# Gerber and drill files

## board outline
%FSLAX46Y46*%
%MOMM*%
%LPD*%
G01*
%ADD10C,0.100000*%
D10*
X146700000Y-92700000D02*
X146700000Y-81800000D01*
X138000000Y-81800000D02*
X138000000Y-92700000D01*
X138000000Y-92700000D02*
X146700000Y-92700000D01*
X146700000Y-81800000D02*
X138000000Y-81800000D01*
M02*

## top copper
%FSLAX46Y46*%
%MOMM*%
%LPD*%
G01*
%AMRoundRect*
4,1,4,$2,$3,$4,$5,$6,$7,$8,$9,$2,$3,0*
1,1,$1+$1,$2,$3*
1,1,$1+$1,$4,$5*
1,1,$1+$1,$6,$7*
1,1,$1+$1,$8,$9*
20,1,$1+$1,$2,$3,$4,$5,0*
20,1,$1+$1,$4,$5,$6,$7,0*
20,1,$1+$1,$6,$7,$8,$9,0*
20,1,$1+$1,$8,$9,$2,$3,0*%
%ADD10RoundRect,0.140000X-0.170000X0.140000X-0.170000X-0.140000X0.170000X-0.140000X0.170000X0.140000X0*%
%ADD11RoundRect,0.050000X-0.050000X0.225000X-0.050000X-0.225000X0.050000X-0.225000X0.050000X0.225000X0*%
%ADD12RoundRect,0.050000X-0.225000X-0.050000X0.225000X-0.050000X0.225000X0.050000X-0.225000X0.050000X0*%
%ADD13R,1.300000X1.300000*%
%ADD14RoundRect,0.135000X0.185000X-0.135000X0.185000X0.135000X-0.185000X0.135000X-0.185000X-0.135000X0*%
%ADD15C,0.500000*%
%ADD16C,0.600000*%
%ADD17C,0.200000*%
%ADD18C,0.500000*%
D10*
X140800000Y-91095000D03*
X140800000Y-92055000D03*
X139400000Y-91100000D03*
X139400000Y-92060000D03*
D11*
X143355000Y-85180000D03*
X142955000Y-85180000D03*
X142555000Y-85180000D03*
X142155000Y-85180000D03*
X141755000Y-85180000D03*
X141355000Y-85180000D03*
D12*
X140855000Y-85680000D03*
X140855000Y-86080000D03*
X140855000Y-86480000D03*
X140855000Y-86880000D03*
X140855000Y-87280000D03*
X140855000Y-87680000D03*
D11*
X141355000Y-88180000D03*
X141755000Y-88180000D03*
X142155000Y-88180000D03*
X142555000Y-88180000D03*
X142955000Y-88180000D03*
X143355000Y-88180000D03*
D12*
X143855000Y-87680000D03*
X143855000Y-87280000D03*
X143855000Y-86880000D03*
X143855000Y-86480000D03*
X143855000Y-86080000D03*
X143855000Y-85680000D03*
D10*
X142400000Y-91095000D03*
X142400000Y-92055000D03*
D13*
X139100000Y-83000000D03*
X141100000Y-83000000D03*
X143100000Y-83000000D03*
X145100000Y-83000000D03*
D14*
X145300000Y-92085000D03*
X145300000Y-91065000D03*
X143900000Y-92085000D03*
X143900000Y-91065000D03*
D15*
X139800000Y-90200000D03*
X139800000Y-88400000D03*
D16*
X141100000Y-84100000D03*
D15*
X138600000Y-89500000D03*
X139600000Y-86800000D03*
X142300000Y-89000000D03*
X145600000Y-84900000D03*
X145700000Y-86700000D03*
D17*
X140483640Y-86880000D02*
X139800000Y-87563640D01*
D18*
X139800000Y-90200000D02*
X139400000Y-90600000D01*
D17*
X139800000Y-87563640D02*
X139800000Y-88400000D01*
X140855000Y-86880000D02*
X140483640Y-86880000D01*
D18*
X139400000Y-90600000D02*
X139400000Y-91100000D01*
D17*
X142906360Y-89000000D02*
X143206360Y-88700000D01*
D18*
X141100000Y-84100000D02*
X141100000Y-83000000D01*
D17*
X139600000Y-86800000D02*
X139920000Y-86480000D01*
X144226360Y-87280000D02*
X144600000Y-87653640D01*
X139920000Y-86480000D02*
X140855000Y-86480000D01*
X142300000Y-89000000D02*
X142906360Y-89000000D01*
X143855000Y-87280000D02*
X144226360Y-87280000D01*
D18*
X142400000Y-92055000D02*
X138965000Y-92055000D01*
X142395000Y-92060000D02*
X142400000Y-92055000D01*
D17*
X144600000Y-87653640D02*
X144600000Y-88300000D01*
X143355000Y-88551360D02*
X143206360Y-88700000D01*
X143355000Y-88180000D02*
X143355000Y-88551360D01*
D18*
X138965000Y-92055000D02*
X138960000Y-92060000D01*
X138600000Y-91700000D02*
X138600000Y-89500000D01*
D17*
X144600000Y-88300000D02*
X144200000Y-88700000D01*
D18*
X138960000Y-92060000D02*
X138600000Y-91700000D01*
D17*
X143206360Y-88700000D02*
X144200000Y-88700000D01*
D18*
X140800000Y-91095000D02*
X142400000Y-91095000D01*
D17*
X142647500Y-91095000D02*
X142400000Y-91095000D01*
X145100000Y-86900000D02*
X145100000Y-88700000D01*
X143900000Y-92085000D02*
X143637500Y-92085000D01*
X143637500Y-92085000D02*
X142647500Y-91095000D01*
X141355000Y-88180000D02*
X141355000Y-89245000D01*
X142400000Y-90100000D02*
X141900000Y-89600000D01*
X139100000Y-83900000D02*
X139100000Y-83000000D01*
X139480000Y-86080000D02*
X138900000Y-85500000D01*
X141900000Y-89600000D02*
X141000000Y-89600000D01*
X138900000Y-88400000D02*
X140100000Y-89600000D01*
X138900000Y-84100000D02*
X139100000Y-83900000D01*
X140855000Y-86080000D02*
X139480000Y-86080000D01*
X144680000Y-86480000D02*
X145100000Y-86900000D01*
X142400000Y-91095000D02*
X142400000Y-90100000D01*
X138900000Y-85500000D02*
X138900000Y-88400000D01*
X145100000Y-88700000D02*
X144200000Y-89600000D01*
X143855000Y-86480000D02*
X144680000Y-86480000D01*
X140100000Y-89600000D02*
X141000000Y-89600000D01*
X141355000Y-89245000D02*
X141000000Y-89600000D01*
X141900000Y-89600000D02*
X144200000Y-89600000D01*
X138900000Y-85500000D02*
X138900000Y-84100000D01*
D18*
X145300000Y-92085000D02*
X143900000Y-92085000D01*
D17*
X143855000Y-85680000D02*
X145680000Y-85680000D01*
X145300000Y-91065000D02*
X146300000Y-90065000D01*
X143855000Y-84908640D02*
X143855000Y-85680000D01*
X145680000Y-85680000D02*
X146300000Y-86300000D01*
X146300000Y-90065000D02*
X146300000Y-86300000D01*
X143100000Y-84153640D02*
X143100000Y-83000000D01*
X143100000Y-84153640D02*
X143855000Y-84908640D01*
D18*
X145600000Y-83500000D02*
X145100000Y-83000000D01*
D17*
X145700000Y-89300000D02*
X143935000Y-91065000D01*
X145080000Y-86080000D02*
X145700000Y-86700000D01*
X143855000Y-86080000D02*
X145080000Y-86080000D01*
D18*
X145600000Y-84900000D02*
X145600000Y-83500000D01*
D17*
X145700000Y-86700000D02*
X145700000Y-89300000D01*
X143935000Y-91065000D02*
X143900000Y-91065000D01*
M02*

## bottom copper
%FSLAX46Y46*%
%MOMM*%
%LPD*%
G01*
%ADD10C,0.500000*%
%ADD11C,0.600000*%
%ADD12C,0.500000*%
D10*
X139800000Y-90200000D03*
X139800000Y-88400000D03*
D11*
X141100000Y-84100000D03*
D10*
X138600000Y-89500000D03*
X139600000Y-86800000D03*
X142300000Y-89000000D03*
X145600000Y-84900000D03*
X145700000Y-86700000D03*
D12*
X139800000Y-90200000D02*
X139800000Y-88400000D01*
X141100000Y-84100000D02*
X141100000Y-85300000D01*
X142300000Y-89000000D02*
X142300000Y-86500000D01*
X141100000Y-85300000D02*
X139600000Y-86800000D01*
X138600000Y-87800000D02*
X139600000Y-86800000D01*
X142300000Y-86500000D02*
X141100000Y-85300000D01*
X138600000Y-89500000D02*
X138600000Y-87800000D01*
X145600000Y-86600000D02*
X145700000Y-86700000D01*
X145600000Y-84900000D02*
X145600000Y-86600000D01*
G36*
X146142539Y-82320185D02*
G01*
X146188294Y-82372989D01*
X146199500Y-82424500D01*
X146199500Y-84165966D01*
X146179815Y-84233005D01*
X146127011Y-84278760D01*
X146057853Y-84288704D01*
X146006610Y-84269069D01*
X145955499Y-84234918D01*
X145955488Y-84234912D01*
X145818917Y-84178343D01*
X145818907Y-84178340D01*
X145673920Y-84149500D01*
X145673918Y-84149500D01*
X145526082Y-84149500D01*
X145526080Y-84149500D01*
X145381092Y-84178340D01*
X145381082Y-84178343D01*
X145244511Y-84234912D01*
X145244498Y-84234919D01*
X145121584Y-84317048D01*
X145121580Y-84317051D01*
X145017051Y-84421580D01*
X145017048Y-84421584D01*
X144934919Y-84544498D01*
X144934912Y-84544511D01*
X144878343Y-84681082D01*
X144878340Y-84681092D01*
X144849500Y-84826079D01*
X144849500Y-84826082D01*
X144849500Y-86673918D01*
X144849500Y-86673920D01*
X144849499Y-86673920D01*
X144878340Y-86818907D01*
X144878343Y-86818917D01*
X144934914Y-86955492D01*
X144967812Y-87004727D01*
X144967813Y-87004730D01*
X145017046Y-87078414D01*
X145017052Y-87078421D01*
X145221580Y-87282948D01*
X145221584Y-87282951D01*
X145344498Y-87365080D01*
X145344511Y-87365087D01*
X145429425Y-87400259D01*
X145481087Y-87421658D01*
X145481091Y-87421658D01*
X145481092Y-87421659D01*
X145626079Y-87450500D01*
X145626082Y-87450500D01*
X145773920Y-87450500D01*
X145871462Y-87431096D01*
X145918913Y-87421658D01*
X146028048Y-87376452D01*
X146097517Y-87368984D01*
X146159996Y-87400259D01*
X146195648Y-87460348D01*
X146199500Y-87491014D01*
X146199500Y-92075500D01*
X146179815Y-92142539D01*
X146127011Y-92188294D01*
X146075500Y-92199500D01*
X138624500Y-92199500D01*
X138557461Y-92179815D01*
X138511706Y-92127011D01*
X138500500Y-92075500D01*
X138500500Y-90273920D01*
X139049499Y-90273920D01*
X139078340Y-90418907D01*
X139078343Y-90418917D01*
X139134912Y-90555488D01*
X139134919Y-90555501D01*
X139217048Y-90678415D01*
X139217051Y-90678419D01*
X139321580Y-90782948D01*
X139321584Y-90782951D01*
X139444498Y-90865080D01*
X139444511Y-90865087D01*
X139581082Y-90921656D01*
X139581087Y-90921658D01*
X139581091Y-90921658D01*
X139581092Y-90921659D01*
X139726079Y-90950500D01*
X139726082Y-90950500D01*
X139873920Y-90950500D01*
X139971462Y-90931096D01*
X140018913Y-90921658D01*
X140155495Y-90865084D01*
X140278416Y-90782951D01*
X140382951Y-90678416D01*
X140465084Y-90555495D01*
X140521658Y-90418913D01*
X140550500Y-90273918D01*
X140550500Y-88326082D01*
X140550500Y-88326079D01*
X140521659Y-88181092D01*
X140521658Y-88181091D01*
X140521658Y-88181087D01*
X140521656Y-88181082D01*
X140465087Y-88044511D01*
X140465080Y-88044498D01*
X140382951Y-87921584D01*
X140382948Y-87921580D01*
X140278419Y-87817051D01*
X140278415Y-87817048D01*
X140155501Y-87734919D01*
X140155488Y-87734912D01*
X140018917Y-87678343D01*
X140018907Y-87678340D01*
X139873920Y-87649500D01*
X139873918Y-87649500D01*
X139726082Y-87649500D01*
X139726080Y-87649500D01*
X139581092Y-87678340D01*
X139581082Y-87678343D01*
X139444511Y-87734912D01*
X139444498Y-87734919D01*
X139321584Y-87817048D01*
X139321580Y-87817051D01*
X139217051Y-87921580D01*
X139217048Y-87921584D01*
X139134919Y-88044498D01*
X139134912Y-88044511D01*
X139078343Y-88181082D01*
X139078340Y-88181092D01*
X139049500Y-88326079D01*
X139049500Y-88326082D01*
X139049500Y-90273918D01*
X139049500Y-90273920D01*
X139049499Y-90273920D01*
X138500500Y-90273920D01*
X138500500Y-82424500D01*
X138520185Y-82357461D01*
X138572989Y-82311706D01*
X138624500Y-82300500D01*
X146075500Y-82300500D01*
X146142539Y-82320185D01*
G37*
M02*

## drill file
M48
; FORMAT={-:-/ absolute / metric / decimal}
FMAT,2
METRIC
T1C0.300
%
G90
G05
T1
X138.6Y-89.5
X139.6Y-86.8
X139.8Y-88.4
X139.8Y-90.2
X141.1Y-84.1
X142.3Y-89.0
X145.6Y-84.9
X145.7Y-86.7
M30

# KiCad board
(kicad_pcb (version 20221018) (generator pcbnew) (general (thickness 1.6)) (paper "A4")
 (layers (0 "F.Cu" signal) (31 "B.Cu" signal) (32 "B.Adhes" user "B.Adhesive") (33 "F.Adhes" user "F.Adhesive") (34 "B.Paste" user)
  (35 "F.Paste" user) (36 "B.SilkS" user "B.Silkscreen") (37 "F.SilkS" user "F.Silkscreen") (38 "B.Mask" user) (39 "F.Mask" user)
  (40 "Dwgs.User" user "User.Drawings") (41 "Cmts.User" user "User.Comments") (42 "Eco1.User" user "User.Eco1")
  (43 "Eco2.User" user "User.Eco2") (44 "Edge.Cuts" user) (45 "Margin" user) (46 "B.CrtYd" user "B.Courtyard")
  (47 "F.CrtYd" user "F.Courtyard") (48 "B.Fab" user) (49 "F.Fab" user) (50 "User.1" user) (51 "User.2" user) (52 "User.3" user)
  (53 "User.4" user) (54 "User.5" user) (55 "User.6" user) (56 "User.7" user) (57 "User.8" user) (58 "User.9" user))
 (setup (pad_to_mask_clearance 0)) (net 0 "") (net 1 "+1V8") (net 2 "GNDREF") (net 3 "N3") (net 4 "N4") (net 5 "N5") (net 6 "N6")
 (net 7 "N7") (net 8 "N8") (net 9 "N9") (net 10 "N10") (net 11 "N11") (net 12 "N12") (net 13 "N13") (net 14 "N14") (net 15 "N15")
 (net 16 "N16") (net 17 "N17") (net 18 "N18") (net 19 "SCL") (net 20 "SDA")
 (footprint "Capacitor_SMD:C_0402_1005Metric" (layer "F.Cu") (at 140.8 91.575 -90)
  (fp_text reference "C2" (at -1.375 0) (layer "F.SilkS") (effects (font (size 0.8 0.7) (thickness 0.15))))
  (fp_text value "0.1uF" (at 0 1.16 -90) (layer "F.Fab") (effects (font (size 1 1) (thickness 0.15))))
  (pad "1" smd roundrect (at -0.48 0 270) (size 0.56 0.62) (layers "F.Cu" "F.Paste" "F.Mask") (roundrect_rratio 0.25) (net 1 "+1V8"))
  (pad "2" smd roundrect (at 0.48 0 270) (size 0.56 0.62) (layers "F.Cu" "F.Paste" "F.Mask") (roundrect_rratio 0.25) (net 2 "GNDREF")))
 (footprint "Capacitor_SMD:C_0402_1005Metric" (layer "F.Cu") (at 139.4 91.58 -90)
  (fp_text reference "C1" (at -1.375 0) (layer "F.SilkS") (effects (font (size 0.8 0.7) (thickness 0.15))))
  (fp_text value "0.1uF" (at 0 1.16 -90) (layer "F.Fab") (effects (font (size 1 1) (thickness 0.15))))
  (pad "1" smd roundrect (at -0.48 0 270) (size 0.56 0.62) (layers "F.Cu" "F.Paste" "F.Mask") (roundrect_rratio 0.25) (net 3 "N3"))
  (pad "2" smd roundrect (at 0.48 0 270) (size 0.56 0.62) (layers "F.Cu" "F.Paste" "F.Mask") (roundrect_rratio 0.25) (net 2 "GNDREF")))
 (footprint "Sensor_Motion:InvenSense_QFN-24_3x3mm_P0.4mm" (layer "F.Cu") (at 142.355 86.68 -90)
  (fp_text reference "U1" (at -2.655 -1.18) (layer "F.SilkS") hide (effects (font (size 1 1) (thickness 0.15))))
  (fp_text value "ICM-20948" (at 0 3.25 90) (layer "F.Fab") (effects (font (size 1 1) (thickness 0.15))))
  (pad "1" smd roundrect (at -1.5 -1 270) (size 0.55 0.2) (layers "F.Cu" "F.Paste" "F.Mask") (roundrect_rratio 0.25) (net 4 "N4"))
  (pad "2" smd roundrect (at -1.5 -0.6 270) (size 0.55 0.2) (layers "F.Cu" "F.Paste" "F.Mask") (roundrect_rratio 0.25) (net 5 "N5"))
  (pad "3" smd roundrect (at -1.5 -0.2 270) (size 0.55 0.2) (layers "F.Cu" "F.Paste" "F.Mask") (roundrect_rratio 0.25) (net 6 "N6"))
  (pad "4" smd roundrect (at -1.5 0.2 270) (size 0.55 0.2) (layers "F.Cu" "F.Paste" "F.Mask") (roundrect_rratio 0.25) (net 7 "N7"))
  (pad "5" smd roundrect (at -1.5 0.6 270) (size 0.55 0.2) (layers "F.Cu" "F.Paste" "F.Mask") (roundrect_rratio 0.25) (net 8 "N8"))
  (pad "6" smd roundrect (at -1.5 1 270) (size 0.55 0.2) (layers "F.Cu" "F.Paste" "F.Mask") (roundrect_rratio 0.25) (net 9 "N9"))
  (pad "7" smd roundrect (at -1 1.5) (size 0.55 0.2) (layers "F.Cu" "F.Paste" "F.Mask") (roundrect_rratio 0.25) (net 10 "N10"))
  (pad "8" smd roundrect (at -0.6 1.5) (size 0.55 0.2) (layers "F.Cu" "F.Paste" "F.Mask") (roundrect_rratio 0.25) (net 1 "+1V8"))
  (pad "9" smd roundrect (at -0.2 1.5) (size 0.55 0.2) (layers "F.Cu" "F.Paste" "F.Mask") (roundrect_rratio 0.25) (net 2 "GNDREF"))
  (pad "10" smd roundrect (at 0.2 1.5) (size 0.55 0.2) (layers "F.Cu" "F.Paste" "F.Mask") (roundrect_rratio 0.25) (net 3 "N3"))
  (pad "11" smd roundrect (at 0.6 1.5) (size 0.55 0.2) (layers "F.Cu" "F.Paste" "F.Mask") (roundrect_rratio 0.25) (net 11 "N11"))
  (pad "12" smd roundrect (at 1 1.5) (size 0.55 0.2) (layers "F.Cu" "F.Paste" "F.Mask") (roundrect_rratio 0.25) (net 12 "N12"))
  (pad "13" smd roundrect (at 1.5 1 270) (size 0.55 0.2) (layers "F.Cu" "F.Paste" "F.Mask") (roundrect_rratio 0.25) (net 1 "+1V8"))
  (pad "14" smd roundrect (at 1.5 0.6 270) (size 0.55 0.2) (layers "F.Cu" "F.Paste" "F.Mask") (roundrect_rratio 0.25) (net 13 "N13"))
  (pad "15" smd roundrect (at 1.5 0.2 270) (size 0.55 0.2) (layers "F.Cu" "F.Paste" "F.Mask") (roundrect_rratio 0.25) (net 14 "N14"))
  (pad "16" smd roundrect (at 1.5 -0.2 270) (size 0.55 0.2) (layers "F.Cu" "F.Paste" "F.Mask") (roundrect_rratio 0.25) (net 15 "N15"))
  (pad "17" smd roundrect (at 1.5 -0.6 270) (size 0.55 0.2) (layers "F.Cu" "F.Paste" "F.Mask") (roundrect_rratio 0.25) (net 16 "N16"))
  (pad "18" smd roundrect (at 1.5 -1 270) (size 0.55 0.2) (layers "F.Cu" "F.Paste" "F.Mask") (roundrect_rratio 0.25) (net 2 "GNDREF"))
  (pad "19" smd roundrect (at 1 -1.5) (size 0.55 0.2) (layers "F.Cu" "F.Paste" "F.Mask") (roundrect_rratio 0.25) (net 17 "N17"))
  (pad "20" smd roundrect (at 0.6 -1.5) (size 0.55 0.2) (layers "F.Cu" "F.Paste" "F.Mask") (roundrect_rratio 0.25) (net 2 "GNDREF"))
  (pad "21" smd roundrect (at 0.2 -1.5) (size 0.55 0.2) (layers "F.Cu" "F.Paste" "F.Mask") (roundrect_rratio 0.25) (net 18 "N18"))
  (pad "22" smd roundrect (at -0.2 -1.5) (size 0.55 0.2) (layers "F.Cu" "F.Paste" "F.Mask") (roundrect_rratio 0.25) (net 1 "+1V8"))
  (pad "23" smd roundrect (at -0.6 -1.5) (size 0.55 0.2) (layers "F.Cu" "F.Paste" "F.Mask") (roundrect_rratio 0.25) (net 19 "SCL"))
  (pad "24" smd roundrect (at -1 -1.5) (size 0.55 0.2) (layers "F.Cu" "F.Paste" "F.Mask") (roundrect_rratio 0.25) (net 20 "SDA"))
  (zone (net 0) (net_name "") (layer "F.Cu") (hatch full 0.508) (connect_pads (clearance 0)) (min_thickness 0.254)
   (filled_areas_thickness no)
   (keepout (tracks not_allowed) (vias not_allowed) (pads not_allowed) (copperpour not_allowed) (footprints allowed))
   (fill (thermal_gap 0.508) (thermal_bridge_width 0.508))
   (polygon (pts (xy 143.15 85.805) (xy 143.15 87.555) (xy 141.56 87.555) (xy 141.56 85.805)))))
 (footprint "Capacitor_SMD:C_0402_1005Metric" (layer "F.Cu") (at 142.4 91.575 -90)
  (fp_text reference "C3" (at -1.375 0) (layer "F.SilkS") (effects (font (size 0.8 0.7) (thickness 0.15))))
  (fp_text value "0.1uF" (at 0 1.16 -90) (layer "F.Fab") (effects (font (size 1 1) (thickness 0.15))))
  (pad "1" smd roundrect (at -0.48 0 270) (size 0.56 0.62) (layers "F.Cu" "F.Paste" "F.Mask") (roundrect_rratio 0.25) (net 1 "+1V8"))
  (pad "2" smd roundrect (at 0.48 0 270) (size 0.56 0.62) (layers "F.Cu" "F.Paste" "F.Mask") (roundrect_rratio 0.25) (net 2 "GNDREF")))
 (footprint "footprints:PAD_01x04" (layer "F.Cu") (at 142.1 83)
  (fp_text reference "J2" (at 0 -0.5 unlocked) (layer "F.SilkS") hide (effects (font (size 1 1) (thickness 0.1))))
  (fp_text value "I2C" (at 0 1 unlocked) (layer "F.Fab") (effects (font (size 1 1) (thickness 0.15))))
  (pad "1" smd rect (at -3 0) (size 1.3 1.3) (layers "F.Cu" "F.Paste" "F.Mask") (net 1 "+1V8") (thermal_bridge_angle 45))
  (pad "2" smd rect (at -1 0) (size 1.3 1.3) (layers "F.Cu" "F.Paste" "F.Mask") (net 2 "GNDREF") (thermal_bridge_angle 45))
  (pad "3" smd rect (at 1 0) (size 1.3 1.3) (layers "F.Cu" "F.Paste" "F.Mask") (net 20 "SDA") (thermal_bridge_angle 45))
  (pad "4" smd rect (at 3 0) (size 1.3 1.3) (layers "F.Cu" "F.Paste" "F.Mask") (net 19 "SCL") (thermal_bridge_angle 45)))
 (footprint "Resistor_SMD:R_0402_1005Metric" (layer "F.Cu") (at 145.3 91.575 90)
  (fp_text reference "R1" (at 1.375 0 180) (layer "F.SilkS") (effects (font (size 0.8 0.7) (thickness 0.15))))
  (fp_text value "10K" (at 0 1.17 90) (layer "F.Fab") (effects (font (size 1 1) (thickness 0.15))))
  (pad "1" smd roundrect (at -0.51 0 90) (size 0.54 0.64) (layers "F.Cu" "F.Paste" "F.Mask") (roundrect_rratio 0.25) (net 1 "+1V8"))
  (pad "2" smd roundrect (at 0.51 0 90) (size 0.54 0.64) (layers "F.Cu" "F.Paste" "F.Mask") (roundrect_rratio 0.25) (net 20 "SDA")))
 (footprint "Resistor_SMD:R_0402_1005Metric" (layer "F.Cu") (at 143.9 91.575 90)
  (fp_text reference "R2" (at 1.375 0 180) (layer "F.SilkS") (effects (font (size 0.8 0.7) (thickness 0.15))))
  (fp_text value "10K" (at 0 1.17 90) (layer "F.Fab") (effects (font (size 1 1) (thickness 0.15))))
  (pad "1" smd roundrect (at -0.51 0 90) (size 0.54 0.64) (layers "F.Cu" "F.Paste" "F.Mask") (roundrect_rratio 0.25) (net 1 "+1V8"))
  (pad "2" smd roundrect (at 0.51 0 90) (size 0.54 0.64) (layers "F.Cu" "F.Paste" "F.Mask") (roundrect_rratio 0.25) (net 19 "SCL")))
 (gr_line (start 146.7 92.7) (end 146.7 81.8) (stroke (width 0.1) (type default)) (layer "Edge.Cuts"))
 (gr_line (start 138 81.8) (end 138 92.7) (stroke (width 0.1) (type default)) (layer "Edge.Cuts"))
 (gr_line (start 138 92.7) (end 146.7 92.7) (stroke (width 0.1) (type default)) (layer "Edge.Cuts"))
 (gr_line (start 146.7 81.8) (end 138 81.8) (stroke (width 0.1) (type default)) (layer "Edge.Cuts"))
 (segment (start 140.48364 86.88) (end 139.8 87.56364) (width 0.2) (layer "F.Cu") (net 3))
 (segment (start 139.8 90.2) (end 139.4 90.6) (width 0.5) (layer "F.Cu") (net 3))
 (segment (start 139.8 87.56364) (end 139.8 88.4) (width 0.2) (layer "F.Cu") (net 3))
 (segment (start 140.855 86.88) (end 140.48364 86.88) (width 0.2) (layer "F.Cu") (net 3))
 (segment (start 139.4 90.6) (end 139.4 91.1) (width 0.5) (layer "F.Cu") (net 3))
 (via (at 139.8 90.2) (size 0.5) (drill 0.3) (layers "F.Cu" "B.Cu") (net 3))
 (via (at 139.8 88.4) (size 0.5) (drill 0.3) (layers "F.Cu" "B.Cu") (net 3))
 (segment (start 139.8 90.2) (end 139.8 88.4) (width 0.5) (layer "B.Cu") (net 3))
 (segment (start 142.90636 89) (end 143.20636 88.7) (width 0.2) (layer "F.Cu") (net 2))
 (segment (start 141.1 84.1) (end 141.1 83) (width 0.5) (layer "F.Cu") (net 2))
 (segment (start 139.6 86.8) (end 139.92 86.48) (width 0.2) (layer "F.Cu") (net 2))
 (segment (start 144.22636 87.28) (end 144.6 87.65364) (width 0.2) (layer "F.Cu") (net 2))
 (segment (start 139.92 86.48) (end 140.855 86.48) (width 0.2) (layer "F.Cu") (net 2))
 (segment (start 142.3 89) (end 142.90636 89) (width 0.2) (layer "F.Cu") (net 2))
 (segment (start 143.855 87.28) (end 144.22636 87.28) (width 0.2) (layer "F.Cu") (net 2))
 (segment (start 142.4 92.055) (end 138.965 92.055) (width 0.5) (layer "F.Cu") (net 2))
 (segment (start 142.395 92.06) (end 142.4 92.055) (width 0.5) (layer "F.Cu") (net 2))
 (segment (start 144.6 87.65364) (end 144.6 88.3) (width 0.2) (layer "F.Cu") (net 2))
 (segment (start 143.355 88.55136) (end 143.20636 88.7) (width 0.2) (layer "F.Cu") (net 2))
 (segment (start 143.355 88.18) (end 143.355 88.55136) (width 0.2) (layer "F.Cu") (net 2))
 (segment (start 138.965 92.055) (end 138.96 92.06) (width 0.5) (layer "F.Cu") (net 2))
 (segment (start 138.6 91.7) (end 138.6 89.5) (width 0.5) (layer "F.Cu") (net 2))
 (segment (start 144.6 88.3) (end 144.2 88.7) (width 0.2) (layer "F.Cu") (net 2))
 (segment (start 138.96 92.06) (end 138.6 91.7) (width 0.5) (layer "F.Cu") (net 2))
 (segment (start 143.20636 88.7) (end 144.2 88.7) (width 0.2) (layer "F.Cu") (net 2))
 (via (at 141.1 84.1) (size 0.6) (drill 0.3) (layers "F.Cu" "B.Cu") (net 2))
 (via (at 138.6 89.5) (size 0.5) (drill 0.3) (layers "F.Cu" "B.Cu") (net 2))
 (via (at 139.6 86.8) (size 0.5) (drill 0.3) (layers "F.Cu" "B.Cu") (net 2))
 (via (at 142.3 89) (size 0.5) (drill 0.3) (layers "F.Cu" "B.Cu") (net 2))
 (segment (start 141.1 84.1) (end 141.1 85.3) (width 0.5) (layer "B.Cu") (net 2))
 (segment (start 142.3 89) (end 142.3 86.5) (width 0.5) (layer "B.Cu") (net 2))
 (segment (start 141.1 85.3) (end 139.6 86.8) (width 0.5) (layer "B.Cu") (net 2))
 (segment (start 138.6 87.8) (end 139.6 86.8) (width 0.5) (layer "B.Cu") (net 2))
 (segment (start 142.3 86.5) (end 141.1 85.3) (width 0.5) (layer "B.Cu") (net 2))
 (segment (start 138.6 89.5) (end 138.6 87.8) (width 0.5) (layer "B.Cu") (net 2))
 (segment (start 140.8 91.095) (end 142.4 91.095) (width 0.5) (layer "F.Cu") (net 1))
 (segment (start 142.6475 91.095) (end 142.4 91.095) (width 0.2) (layer "F.Cu") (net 1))
 (segment (start 145.1 86.9) (end 145.1 88.7) (width 0.2) (layer "F.Cu") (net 1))
 (segment (start 143.9 92.085) (end 143.6375 92.085) (width 0.2) (layer "F.Cu") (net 1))
 (segment (start 143.6375 92.085) (end 142.6475 91.095) (width 0.2) (layer "F.Cu") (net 1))
 (segment (start 141.355 88.18) (end 141.355 89.245) (width 0.2) (layer "F.Cu") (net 1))
 (segment (start 142.4 90.1) (end 141.9 89.6) (width 0.2) (layer "F.Cu") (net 1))
 (segment (start 139.1 83.9) (end 139.1 83) (width 0.2) (layer "F.Cu") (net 1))
 (segment (start 139.48 86.08) (end 138.9 85.5) (width 0.2) (layer "F.Cu") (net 1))
 (segment (start 141.9 89.6) (end 141 89.6) (width 0.2) (layer "F.Cu") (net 1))
 (segment (start 138.9 88.4) (end 140.1 89.6) (width 0.2) (layer "F.Cu") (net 1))
 (segment (start 138.9 84.1) (end 139.1 83.9) (width 0.2) (layer "F.Cu") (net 1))
 (segment (start 140.855 86.08) (end 139.48 86.08) (width 0.2) (layer "F.Cu") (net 1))
 (segment (start 144.68 86.48) (end 145.1 86.9) (width 0.2) (layer "F.Cu") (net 1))
 (segment (start 142.4 91.095) (end 142.4 90.1) (width 0.2) (layer "F.Cu") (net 1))
 (segment (start 138.9 85.5) (end 138.9 88.4) (width 0.2) (layer "F.Cu") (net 1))
 (segment (start 145.1 88.7) (end 144.2 89.6) (width 0.2) (layer "F.Cu") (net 1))
 (segment (start 143.855 86.48) (end 144.68 86.48) (width 0.2) (layer "F.Cu") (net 1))
 (segment (start 140.1 89.6) (end 141 89.6) (width 0.2) (layer "F.Cu") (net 1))
 (segment (start 141.355 89.245) (end 141 89.6) (width 0.2) (layer "F.Cu") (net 1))
 (segment (start 141.9 89.6) (end 144.2 89.6) (width 0.2) (layer "F.Cu") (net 1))
 (segment (start 138.9 85.5) (end 138.9 84.1) (width 0.2) (layer "F.Cu") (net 1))
 (segment (start 145.3 92.085) (end 143.9 92.085) (width 0.5) (layer "F.Cu") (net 1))
 (segment (start 143.855 85.68) (end 145.68 85.68) (width 0.2) (layer "F.Cu") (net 20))
 (segment (start 145.3 91.065) (end 146.3 90.065) (width 0.2) (layer "F.Cu") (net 20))
 (segment (start 143.855 84.90864) (end 143.855 85.68) (width 0.2) (layer "F.Cu") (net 20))
 (segment (start 145.68 85.68) (end 146.3 86.3) (width 0.2) (layer "F.Cu") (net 20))
 (segment (start 146.3 90.065) (end 146.3 86.3) (width 0.2) (layer "F.Cu") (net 20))
 (segment (start 143.1 84.15364) (end 143.1 83) (width 0.2) (layer "F.Cu") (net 20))
 (segment (start 143.1 84.15364) (end 143.855 84.90864) (width 0.2) (layer "F.Cu") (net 20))
 (segment (start 145.6 83.5) (end 145.1 83) (width 0.5) (layer "F.Cu") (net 19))
 (segment (start 145.7 89.3) (end 143.935 91.065) (width 0.2) (layer "F.Cu") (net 19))
 (segment (start 145.08 86.08) (end 145.7 86.7) (width 0.2) (layer "F.Cu") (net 19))
 (segment (start 143.855 86.08) (end 145.08 86.08) (width 0.2) (layer "F.Cu") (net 19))
 (segment (start 145.6 84.9) (end 145.6 83.5) (width 0.5) (layer "F.Cu") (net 19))
 (segment (start 145.7 86.7) (end 145.7 89.3) (width 0.2) (layer "F.Cu") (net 19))
 (segment (start 143.935 91.065) (end 143.9 91.065) (width 0.2) (layer "F.Cu") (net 19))
 (via (at 145.6 84.9) (size 0.5) (drill 0.3) (layers "F.Cu" "B.Cu") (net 19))
 (via (at 145.7 86.7) (size 0.5) (drill 0.3) (layers "F.Cu" "B.Cu") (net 19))
 (segment (start 145.6 86.6) (end 145.7 86.7) (width 0.5) (layer "B.Cu") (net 19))
 (segment (start 145.6 84.9) (end 145.6 86.6) (width 0.5) (layer "B.Cu") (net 19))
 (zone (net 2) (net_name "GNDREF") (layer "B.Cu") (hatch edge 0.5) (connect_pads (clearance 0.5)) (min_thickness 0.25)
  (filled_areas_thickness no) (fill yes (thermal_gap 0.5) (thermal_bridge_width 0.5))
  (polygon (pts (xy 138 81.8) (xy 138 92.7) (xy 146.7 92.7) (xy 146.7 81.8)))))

